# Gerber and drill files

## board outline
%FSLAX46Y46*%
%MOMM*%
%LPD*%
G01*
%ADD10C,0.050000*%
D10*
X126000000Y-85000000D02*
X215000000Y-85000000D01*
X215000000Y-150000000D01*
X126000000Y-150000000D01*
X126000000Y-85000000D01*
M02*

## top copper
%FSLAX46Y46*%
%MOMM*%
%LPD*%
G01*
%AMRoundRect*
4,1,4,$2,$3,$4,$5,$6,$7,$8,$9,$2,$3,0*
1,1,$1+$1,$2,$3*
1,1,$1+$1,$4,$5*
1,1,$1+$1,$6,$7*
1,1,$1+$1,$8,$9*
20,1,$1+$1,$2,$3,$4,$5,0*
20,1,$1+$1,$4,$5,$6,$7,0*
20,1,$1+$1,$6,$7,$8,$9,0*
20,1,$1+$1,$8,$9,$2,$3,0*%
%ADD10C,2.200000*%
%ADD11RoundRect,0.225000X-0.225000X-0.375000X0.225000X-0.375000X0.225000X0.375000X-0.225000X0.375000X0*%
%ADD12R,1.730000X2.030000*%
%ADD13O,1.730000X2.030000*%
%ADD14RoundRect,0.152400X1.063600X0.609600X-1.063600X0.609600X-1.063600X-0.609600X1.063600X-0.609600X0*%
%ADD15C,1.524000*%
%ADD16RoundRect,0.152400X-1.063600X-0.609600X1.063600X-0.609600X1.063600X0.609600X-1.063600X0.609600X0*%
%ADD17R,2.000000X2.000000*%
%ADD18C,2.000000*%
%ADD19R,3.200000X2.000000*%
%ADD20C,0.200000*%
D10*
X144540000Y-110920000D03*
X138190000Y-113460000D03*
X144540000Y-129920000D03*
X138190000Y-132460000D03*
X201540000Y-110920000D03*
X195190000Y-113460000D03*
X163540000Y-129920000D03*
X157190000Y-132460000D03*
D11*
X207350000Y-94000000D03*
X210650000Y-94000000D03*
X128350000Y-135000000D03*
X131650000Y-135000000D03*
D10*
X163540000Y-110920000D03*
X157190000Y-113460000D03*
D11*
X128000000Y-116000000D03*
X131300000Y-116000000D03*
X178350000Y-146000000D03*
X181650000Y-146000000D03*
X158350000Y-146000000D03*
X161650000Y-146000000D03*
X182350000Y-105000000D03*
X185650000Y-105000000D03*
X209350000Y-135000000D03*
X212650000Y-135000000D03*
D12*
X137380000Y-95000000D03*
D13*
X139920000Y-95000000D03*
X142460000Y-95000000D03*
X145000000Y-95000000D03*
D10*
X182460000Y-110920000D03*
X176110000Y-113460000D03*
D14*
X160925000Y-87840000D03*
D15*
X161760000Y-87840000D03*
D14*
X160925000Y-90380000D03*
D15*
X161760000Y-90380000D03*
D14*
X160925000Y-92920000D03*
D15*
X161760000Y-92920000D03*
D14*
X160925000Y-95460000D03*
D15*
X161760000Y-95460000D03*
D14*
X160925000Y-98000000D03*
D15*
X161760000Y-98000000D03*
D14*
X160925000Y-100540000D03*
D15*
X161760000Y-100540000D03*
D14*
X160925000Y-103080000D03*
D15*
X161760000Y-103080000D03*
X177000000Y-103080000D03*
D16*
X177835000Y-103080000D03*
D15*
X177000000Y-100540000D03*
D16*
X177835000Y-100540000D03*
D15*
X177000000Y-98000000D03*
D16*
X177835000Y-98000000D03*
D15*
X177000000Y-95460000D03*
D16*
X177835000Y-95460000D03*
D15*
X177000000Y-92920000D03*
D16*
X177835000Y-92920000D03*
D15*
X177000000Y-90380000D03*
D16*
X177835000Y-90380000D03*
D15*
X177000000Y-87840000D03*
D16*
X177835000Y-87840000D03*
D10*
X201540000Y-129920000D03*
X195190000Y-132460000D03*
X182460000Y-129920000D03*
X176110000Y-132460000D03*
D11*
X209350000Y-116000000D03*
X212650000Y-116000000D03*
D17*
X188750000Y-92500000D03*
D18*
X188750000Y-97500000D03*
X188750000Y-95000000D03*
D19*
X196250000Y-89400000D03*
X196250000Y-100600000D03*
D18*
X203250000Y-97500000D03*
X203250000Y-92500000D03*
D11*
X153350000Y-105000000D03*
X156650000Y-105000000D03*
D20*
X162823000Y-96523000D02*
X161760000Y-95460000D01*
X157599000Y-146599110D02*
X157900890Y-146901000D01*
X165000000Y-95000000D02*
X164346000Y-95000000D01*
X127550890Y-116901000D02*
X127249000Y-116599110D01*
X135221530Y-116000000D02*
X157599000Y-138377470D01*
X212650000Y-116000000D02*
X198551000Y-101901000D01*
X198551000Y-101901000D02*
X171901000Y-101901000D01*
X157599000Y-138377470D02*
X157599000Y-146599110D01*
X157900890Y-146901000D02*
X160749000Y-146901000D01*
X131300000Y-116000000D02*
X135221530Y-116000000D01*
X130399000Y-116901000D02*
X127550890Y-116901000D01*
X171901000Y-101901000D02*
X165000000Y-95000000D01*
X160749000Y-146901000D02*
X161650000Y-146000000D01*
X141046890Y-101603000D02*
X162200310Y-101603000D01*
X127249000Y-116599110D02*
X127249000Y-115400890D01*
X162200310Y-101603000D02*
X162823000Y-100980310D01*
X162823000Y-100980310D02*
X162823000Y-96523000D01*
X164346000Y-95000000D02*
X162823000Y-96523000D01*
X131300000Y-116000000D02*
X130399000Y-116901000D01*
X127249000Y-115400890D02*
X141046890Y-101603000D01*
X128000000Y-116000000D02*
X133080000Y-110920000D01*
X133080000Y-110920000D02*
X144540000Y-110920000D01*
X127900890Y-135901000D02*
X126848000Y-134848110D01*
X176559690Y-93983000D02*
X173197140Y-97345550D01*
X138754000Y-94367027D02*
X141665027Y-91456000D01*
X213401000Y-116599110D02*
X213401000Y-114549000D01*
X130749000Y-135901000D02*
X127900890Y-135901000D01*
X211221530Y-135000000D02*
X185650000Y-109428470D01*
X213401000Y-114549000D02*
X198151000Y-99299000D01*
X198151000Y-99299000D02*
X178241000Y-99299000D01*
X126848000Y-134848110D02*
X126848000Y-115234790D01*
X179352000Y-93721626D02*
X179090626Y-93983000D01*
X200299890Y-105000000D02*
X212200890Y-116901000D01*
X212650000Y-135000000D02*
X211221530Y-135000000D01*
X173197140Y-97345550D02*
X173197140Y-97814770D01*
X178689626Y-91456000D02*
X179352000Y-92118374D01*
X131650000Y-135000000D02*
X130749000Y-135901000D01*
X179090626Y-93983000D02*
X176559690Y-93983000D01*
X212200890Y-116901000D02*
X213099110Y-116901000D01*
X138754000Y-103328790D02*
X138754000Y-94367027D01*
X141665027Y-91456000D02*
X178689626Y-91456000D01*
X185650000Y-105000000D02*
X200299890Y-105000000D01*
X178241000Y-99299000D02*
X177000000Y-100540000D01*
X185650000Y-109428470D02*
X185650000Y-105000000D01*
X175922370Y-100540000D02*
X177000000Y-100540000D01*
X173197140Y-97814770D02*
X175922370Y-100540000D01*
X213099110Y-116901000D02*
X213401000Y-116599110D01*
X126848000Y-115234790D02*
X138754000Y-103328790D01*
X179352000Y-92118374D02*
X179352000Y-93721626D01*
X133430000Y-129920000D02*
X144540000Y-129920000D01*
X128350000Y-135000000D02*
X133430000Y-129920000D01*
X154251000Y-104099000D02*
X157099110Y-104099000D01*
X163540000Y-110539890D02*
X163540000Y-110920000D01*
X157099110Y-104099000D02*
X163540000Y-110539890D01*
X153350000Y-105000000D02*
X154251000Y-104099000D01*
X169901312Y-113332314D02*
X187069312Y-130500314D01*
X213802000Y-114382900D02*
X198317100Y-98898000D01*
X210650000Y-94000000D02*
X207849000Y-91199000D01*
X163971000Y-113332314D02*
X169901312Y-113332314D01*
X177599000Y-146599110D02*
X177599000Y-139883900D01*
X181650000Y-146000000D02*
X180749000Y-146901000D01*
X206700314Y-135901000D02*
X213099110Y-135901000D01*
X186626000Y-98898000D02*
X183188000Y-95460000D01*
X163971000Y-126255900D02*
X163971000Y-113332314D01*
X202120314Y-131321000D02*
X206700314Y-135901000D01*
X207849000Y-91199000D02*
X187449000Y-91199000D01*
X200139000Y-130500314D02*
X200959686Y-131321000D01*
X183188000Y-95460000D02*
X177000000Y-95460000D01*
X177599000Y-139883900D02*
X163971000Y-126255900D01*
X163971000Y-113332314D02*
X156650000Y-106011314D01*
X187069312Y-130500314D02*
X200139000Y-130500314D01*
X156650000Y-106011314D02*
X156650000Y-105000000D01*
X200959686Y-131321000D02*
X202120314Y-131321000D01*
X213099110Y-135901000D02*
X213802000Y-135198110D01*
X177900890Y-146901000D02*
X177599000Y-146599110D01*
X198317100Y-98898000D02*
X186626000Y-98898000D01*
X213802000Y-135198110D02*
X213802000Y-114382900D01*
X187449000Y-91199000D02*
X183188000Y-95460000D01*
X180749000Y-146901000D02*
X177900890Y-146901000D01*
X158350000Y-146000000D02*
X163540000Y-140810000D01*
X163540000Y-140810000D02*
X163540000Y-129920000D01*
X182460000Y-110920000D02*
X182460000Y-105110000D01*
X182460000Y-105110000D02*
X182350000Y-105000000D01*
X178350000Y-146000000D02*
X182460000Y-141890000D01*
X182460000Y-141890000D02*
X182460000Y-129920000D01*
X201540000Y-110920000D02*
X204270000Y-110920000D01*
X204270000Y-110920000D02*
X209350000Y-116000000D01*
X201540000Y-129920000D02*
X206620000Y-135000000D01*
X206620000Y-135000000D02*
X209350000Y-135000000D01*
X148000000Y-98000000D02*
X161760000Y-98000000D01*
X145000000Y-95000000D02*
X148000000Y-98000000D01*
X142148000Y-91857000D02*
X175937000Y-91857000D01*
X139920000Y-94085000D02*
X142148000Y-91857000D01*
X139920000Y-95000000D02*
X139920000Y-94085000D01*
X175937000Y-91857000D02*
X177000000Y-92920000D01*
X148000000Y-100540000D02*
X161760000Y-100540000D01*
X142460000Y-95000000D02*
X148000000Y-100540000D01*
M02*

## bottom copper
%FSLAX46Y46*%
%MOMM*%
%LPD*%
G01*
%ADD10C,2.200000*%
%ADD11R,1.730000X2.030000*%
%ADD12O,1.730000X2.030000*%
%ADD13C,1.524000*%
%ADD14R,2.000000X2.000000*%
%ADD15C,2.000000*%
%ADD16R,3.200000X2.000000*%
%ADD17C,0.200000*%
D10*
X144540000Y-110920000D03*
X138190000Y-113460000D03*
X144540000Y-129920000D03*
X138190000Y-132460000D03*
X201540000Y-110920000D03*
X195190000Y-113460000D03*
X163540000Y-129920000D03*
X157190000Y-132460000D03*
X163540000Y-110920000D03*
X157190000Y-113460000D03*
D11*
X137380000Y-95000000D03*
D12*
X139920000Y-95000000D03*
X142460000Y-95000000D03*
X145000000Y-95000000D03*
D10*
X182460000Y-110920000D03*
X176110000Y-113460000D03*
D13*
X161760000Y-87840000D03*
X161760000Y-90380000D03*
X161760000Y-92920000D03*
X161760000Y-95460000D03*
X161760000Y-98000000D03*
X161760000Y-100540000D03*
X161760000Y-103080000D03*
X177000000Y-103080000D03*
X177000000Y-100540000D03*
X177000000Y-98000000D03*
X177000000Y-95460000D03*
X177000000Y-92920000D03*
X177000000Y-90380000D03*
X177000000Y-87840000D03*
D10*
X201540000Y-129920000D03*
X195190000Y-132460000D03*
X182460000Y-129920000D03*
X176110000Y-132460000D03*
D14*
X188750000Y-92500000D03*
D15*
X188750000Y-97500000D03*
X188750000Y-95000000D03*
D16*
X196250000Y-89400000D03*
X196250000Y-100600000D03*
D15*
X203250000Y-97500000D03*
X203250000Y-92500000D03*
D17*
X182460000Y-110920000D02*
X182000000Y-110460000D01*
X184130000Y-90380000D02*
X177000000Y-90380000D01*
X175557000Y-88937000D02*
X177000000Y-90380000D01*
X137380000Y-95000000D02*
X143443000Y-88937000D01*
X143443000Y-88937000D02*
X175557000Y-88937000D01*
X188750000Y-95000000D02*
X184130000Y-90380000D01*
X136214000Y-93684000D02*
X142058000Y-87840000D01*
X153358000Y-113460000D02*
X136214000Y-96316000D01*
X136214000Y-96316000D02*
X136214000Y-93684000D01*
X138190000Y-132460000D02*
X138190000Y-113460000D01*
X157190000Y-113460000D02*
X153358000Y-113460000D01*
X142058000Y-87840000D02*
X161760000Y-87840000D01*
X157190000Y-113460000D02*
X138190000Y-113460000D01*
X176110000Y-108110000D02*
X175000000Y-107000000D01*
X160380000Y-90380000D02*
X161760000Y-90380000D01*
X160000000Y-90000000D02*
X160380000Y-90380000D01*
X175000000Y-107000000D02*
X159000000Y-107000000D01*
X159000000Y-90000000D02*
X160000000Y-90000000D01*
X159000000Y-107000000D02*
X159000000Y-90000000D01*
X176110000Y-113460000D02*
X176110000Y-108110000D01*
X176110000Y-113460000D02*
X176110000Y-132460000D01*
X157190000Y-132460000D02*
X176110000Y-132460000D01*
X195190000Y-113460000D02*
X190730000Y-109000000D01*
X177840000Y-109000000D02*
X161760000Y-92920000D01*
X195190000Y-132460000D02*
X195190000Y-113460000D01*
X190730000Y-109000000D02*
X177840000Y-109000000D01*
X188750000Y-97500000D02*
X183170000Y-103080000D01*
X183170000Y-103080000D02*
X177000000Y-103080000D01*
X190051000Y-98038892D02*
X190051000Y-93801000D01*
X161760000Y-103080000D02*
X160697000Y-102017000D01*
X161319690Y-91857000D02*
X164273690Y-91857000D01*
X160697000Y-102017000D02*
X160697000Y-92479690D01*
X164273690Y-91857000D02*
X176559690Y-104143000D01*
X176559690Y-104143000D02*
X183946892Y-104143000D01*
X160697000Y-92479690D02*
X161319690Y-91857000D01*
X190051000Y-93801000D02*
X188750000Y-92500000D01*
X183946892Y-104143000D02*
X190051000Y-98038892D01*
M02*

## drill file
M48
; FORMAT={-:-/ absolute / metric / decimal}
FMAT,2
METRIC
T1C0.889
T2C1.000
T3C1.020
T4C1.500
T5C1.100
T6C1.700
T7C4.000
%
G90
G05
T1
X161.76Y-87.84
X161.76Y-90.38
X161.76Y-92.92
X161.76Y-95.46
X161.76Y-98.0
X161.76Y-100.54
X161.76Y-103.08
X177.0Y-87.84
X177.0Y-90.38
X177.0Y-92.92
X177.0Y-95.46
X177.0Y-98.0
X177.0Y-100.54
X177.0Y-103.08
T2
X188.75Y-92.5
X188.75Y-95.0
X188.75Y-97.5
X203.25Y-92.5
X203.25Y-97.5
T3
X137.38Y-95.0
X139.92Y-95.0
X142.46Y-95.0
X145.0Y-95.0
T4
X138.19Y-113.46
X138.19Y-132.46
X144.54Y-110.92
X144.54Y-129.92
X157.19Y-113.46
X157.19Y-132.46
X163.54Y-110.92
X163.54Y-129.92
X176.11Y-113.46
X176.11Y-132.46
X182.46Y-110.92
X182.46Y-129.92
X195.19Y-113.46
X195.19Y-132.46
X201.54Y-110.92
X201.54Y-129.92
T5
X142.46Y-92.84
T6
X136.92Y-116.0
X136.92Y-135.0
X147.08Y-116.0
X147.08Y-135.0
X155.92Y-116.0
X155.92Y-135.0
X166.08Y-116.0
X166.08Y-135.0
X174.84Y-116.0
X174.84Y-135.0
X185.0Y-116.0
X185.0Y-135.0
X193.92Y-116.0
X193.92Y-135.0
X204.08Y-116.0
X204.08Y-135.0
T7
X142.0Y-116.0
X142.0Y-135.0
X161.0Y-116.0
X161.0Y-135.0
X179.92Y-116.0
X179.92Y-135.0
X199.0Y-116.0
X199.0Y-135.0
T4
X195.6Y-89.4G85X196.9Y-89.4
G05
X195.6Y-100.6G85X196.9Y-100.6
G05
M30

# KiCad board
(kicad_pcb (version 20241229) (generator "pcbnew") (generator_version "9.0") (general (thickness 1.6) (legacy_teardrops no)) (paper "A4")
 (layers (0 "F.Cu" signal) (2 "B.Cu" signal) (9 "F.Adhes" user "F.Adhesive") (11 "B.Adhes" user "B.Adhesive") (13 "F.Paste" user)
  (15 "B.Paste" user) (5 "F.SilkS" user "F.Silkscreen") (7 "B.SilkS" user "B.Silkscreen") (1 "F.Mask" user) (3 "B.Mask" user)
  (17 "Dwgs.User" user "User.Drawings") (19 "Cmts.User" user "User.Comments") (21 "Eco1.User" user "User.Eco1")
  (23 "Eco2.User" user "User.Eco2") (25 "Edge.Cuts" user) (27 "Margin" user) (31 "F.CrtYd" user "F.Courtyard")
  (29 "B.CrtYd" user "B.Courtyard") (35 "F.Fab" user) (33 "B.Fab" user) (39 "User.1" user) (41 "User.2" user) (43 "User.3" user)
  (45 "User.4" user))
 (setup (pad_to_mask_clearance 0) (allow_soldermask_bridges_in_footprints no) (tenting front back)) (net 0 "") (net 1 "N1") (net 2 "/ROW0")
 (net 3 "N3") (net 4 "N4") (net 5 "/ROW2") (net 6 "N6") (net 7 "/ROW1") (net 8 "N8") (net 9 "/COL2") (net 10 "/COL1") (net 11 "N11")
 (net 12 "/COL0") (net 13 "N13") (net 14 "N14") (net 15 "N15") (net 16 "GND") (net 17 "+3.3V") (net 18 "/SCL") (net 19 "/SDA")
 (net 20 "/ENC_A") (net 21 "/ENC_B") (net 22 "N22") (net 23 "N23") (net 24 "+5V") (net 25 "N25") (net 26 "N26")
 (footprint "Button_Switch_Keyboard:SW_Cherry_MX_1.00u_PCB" (layer "F.Cu") (at 144.54 110.92)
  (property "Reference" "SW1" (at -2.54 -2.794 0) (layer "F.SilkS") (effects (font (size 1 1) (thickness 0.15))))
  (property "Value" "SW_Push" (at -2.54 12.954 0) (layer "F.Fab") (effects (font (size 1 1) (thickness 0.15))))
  (pad "" np_thru_hole circle (at -7.62 5.08) (size 1.7 1.7) (drill 1.7) (layers "*.Cu" "*.Mask"))
  (pad "" np_thru_hole circle (at -2.54 5.08) (size 4 4) (drill 4) (layers "*.Cu" "*.Mask"))
  (pad "" np_thru_hole circle (at 2.54 5.08) (size 1.7 1.7) (drill 1.7) (layers "*.Cu" "*.Mask"))
  (pad "1" thru_hole circle (at 0 0) (size 2.2 2.2) (drill 1.5) (layers "*.Cu" "*.Mask") (remove_unused_layers no) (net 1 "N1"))
  (pad "2" thru_hole circle (at -6.35 2.54) (size 2.2 2.2) (drill 1.5) (layers "*.Cu" "*.Mask") (remove_unused_layers no) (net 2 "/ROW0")))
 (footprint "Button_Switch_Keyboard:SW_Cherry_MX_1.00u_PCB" (layer "F.Cu") (at 144.54 129.92)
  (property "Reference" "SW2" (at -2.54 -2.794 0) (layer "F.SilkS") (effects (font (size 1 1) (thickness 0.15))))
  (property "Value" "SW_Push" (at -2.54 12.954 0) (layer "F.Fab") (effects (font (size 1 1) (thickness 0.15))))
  (pad "" np_thru_hole circle (at -7.62 5.08) (size 1.7 1.7) (drill 1.7) (layers "*.Cu" "*.Mask"))
  (pad "" np_thru_hole circle (at -2.54 5.08) (size 4 4) (drill 4) (layers "*.Cu" "*.Mask"))
  (pad "" np_thru_hole circle (at 2.54 5.08) (size 1.7 1.7) (drill 1.7) (layers "*.Cu" "*.Mask"))
  (pad "1" thru_hole circle (at 0 0) (size 2.2 2.2) (drill 1.5) (layers "*.Cu" "*.Mask") (remove_unused_layers no) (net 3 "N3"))
  (pad "2" thru_hole circle (at -6.35 2.54) (size 2.2 2.2) (drill 1.5) (layers "*.Cu" "*.Mask") (remove_unused_layers no) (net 2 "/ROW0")))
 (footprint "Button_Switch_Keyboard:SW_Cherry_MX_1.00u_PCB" (layer "F.Cu") (at 201.54 110.92)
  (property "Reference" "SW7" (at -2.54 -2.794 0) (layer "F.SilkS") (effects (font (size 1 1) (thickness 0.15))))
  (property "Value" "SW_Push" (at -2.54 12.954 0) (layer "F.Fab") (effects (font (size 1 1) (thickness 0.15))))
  (pad "" np_thru_hole circle (at -7.62 5.08) (size 1.7 1.7) (drill 1.7) (layers "*.Cu" "*.Mask"))
  (pad "" np_thru_hole circle (at -2.54 5.08) (size 4 4) (drill 4) (layers "*.Cu" "*.Mask"))
  (pad "" np_thru_hole circle (at 2.54 5.08) (size 1.7 1.7) (drill 1.7) (layers "*.Cu" "*.Mask"))
  (pad "1" thru_hole circle (at 0 0) (size 2.2 2.2) (drill 1.5) (layers "*.Cu" "*.Mask") (remove_unused_layers no) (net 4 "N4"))
  (pad "2" thru_hole circle (at -6.35 2.54) (size 2.2 2.2) (drill 1.5) (layers "*.Cu" "*.Mask") (remove_unused_layers no) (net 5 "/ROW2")))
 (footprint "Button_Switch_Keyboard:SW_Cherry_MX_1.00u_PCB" (layer "F.Cu") (at 163.54 129.92)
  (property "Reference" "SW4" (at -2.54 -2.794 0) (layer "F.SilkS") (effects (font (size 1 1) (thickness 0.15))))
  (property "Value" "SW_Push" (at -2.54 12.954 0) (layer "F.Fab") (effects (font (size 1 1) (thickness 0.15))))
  (pad "" np_thru_hole circle (at -7.62 5.08) (size 1.7 1.7) (drill 1.7) (layers "*.Cu" "*.Mask"))
  (pad "" np_thru_hole circle (at -2.54 5.08) (size 4 4) (drill 4) (layers "*.Cu" "*.Mask"))
  (pad "" np_thru_hole circle (at 2.54 5.08) (size 1.7 1.7) (drill 1.7) (layers "*.Cu" "*.Mask"))
  (pad "1" thru_hole circle (at 0 0) (size 2.2 2.2) (drill 1.5) (layers "*.Cu" "*.Mask") (remove_unused_layers no) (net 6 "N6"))
  (pad "2" thru_hole circle (at -6.35 2.54) (size 2.2 2.2) (drill 1.5) (layers "*.Cu" "*.Mask") (remove_unused_layers no) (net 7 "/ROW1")))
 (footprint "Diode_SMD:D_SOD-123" (layer "F.Cu") (at 209 94)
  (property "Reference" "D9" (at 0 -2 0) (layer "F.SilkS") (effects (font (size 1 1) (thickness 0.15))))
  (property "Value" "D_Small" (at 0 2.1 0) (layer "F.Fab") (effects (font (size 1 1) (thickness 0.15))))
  (pad "1" smd roundrect (at -1.65 0) (size 0.9 1.2) (layers "F.Cu" "F.Mask" "F.Paste") (roundrect_rratio 0.25) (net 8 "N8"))
  (pad "2" smd roundrect (at 1.65 0) (size 0.9 1.2) (layers "F.Cu" "F.Mask" "F.Paste") (roundrect_rratio 0.25) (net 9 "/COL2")))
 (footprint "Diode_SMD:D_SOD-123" (layer "F.Cu") (at 130 135)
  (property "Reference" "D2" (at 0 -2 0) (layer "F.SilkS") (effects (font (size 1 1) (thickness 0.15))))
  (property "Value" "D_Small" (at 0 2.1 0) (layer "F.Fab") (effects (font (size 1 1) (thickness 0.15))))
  (pad "1" smd roundrect (at -1.65 0) (size 0.9 1.2) (layers "F.Cu" "F.Mask" "F.Paste") (roundrect_rratio 0.25) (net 3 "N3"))
  (pad "2" smd roundrect (at 1.65 0) (size 0.9 1.2) (layers "F.Cu" "F.Mask" "F.Paste") (roundrect_rratio 0.25) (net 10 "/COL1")))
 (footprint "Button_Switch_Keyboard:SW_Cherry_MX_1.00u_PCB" (layer "F.Cu") (at 163.54 110.92)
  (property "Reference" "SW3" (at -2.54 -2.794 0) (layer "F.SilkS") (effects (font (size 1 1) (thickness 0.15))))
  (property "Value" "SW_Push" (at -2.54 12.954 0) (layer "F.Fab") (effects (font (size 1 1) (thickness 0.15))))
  (pad "" np_thru_hole circle (at -7.62 5.08) (size 1.7 1.7) (drill 1.7) (layers "*.Cu" "*.Mask"))
  (pad "" np_thru_hole circle (at -2.54 5.08) (size 4 4) (drill 4) (layers "*.Cu" "*.Mask"))
  (pad "" np_thru_hole circle (at 2.54 5.08) (size 1.7 1.7) (drill 1.7) (layers "*.Cu" "*.Mask"))
  (pad "1" thru_hole circle (at 0 0) (size 2.2 2.2) (drill 1.5) (layers "*.Cu" "*.Mask") (remove_unused_layers no) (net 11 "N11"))
  (pad "2" thru_hole circle (at -6.35 2.54) (size 2.2 2.2) (drill 1.5) (layers "*.Cu" "*.Mask") (remove_unused_layers no) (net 2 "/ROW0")))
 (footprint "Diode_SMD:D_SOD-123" (layer "F.Cu") (at 129.65 116)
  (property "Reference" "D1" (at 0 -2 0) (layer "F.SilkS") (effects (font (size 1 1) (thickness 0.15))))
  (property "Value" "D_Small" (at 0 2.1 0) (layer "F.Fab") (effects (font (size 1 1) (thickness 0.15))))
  (pad "1" smd roundrect (at -1.65 0) (size 0.9 1.2) (layers "F.Cu" "F.Mask" "F.Paste") (roundrect_rratio 0.25) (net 1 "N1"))
  (pad "2" smd roundrect (at 1.65 0) (size 0.9 1.2) (layers "F.Cu" "F.Mask" "F.Paste") (roundrect_rratio 0.25) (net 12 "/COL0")))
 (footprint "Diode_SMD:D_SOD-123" (layer "F.Cu") (at 180 146)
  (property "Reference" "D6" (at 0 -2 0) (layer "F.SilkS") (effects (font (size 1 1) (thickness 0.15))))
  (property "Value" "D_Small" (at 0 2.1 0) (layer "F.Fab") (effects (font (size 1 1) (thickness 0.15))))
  (pad "1" smd roundrect (at -1.65 0) (size 0.9 1.2) (layers "F.Cu" "F.Mask" "F.Paste") (roundrect_rratio 0.25) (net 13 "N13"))
  (pad "2" smd roundrect (at 1.65 0) (size 0.9 1.2) (layers "F.Cu" "F.Mask" "F.Paste") (roundrect_rratio 0.25) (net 9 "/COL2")))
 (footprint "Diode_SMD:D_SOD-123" (layer "F.Cu") (at 160 146)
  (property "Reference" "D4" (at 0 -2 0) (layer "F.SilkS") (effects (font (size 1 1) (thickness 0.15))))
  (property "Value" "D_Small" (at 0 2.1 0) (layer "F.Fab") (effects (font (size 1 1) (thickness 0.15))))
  (pad "1" smd roundrect (at -1.65 0) (size 0.9 1.2) (layers "F.Cu" "F.Mask" "F.Paste") (roundrect_rratio 0.25) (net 6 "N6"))
  (pad "2" smd roundrect (at 1.65 0) (size 0.9 1.2) (layers "F.Cu" "F.Mask" "F.Paste") (roundrect_rratio 0.25) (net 12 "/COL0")))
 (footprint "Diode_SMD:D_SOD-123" (layer "F.Cu") (at 184 105)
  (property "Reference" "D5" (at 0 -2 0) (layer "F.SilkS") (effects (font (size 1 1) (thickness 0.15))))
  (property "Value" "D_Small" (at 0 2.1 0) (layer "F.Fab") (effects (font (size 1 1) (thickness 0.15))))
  (pad "1" smd roundrect (at -1.65 0) (size 0.9 1.2) (layers "F.Cu" "F.Mask" "F.Paste") (roundrect_rratio 0.25) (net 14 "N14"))
  (pad "2" smd roundrect (at 1.65 0) (size 0.9 1.2) (layers "F.Cu" "F.Mask" "F.Paste") (roundrect_rratio 0.25) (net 10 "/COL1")))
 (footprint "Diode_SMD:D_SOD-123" (layer "F.Cu") (at 211 135)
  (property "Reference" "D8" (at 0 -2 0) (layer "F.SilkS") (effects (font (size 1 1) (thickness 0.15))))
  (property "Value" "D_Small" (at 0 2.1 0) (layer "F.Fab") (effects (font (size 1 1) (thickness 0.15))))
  (pad "1" smd roundrect (at -1.65 0) (size 0.9 1.2) (layers "F.Cu" "F.Mask" "F.Paste") (roundrect_rratio 0.25) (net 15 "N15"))
  (pad "2" smd roundrect (at 1.65 0) (size 0.9 1.2) (layers "F.Cu" "F.Mask" "F.Paste") (roundrect_rratio 0.25) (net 10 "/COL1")))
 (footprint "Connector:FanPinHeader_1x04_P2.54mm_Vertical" (layer "F.Cu") (at 137.38 95)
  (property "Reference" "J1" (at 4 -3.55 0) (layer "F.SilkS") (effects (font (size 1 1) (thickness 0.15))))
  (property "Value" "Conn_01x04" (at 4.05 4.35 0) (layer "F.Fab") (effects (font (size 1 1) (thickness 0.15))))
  (pad "" np_thru_hole circle (at 5.08 -2.16 90) (size 1.1 1.1) (drill 1.1) (layers "*.Cu" "*.Mask"))
  (pad "1" thru_hole rect (at 0 0 90) (size 2.03 1.73) (drill 1.02) (layers "*.Cu" "*.Mask") (remove_unused_layers no) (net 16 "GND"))
  (pad "2" thru_hole oval (at 2.54 0 90) (size 2.03 1.73) (drill 1.02) (layers "*.Cu" "*.Mask") (remove_unused_layers no) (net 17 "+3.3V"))
  (pad "3" thru_hole oval (at 5.08 0 90) (size 2.03 1.73) (drill 1.02) (layers "*.Cu" "*.Mask") (remove_unused_layers no) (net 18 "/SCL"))
  (pad "4" thru_hole oval (at 7.62 0 90) (size 2.03 1.73) (drill 1.02) (layers "*.Cu" "*.Mask") (remove_unused_layers no) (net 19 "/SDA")))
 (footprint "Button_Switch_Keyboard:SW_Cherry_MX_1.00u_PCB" (layer "F.Cu") (at 182.46 110.92)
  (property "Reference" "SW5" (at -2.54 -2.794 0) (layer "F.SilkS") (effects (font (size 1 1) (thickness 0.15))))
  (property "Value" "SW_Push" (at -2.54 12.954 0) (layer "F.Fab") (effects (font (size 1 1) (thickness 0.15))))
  (pad "" np_thru_hole circle (at -7.62 5.08) (size 1.7 1.7) (drill 1.7) (layers "*.Cu" "*.Mask"))
  (pad "" np_thru_hole circle (at -2.54 5.08) (size 4 4) (drill 4) (layers "*.Cu" "*.Mask"))
  (pad "" np_thru_hole circle (at 2.54 5.08) (size 1.7 1.7) (drill 1.7) (layers "*.Cu" "*.Mask"))
  (pad "1" thru_hole circle (at 0 0) (size 2.2 2.2) (drill 1.5) (layers "*.Cu" "*.Mask") (remove_unused_layers no) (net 14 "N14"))
  (pad "2" thru_hole circle (at -6.35 2.54) (size 2.2 2.2) (drill 1.5) (layers "*.Cu" "*.Mask") (remove_unused_layers no) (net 7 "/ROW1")))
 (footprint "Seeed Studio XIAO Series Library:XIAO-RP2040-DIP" (layer "F.Cu") (at 169.38 95.46)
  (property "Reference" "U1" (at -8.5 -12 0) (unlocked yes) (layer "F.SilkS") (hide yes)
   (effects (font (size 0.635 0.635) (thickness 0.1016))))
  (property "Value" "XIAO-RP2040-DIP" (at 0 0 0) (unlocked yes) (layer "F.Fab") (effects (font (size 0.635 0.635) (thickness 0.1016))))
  (pad "1" smd roundrect (at -8.455 -7.62 180) (size 2.432 1.524) (layers "F.Cu" "F.Mask") (roundrect_rratio 0.1) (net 2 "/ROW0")
   (thermal_bridge_angle 45))
  (pad "1" thru_hole circle (at -7.62 -7.62 180) (size 1.524 1.524) (drill 0.889) (layers "*.Cu" "*.Mask") (remove_unused_layers no)
   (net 2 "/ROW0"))
  (pad "2" smd roundrect (at -8.455 -5.08 180) (size 2.432 1.524) (layers "F.Cu" "F.Mask") (roundrect_rratio 0.1) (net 7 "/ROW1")
   (thermal_bridge_angle 45))
  (pad "2" thru_hole circle (at -7.62 -5.08 180) (size 1.524 1.524) (drill 0.889) (layers "*.Cu" "*.Mask") (remove_unused_layers no)
   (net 7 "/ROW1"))
  (pad "3" smd roundrect (at -8.455 -2.54 180) (size 2.432 1.524) (layers "F.Cu" "F.Mask") (roundrect_rratio 0.1) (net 5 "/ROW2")
   (thermal_bridge_angle 45))
  (pad "3" thru_hole circle (at -7.62 -2.54 180) (size 1.524 1.524) (drill 0.889) (layers "*.Cu" "*.Mask") (remove_unused_layers no)
   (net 5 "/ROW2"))
  (pad "4" smd roundrect (at -8.455 0 180) (size 2.432 1.524) (layers "F.Cu" "F.Mask") (roundrect_rratio 0.1) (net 12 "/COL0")
   (thermal_bridge_angle 45))
  (pad "4" thru_hole circle (at -7.62 0 180) (size 1.524 1.524) (drill 0.889) (layers "*.Cu" "*.Mask") (remove_unused_layers no)
   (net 12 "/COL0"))
  (pad "5" smd roundrect (at -8.455 2.54 180) (size 2.432 1.524) (layers "F.Cu" "F.Mask") (roundrect_rratio 0.1) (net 19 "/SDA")
   (thermal_bridge_angle 45))
  (pad "5" thru_hole circle (at -7.62 2.54 180) (size 1.524 1.524) (drill 0.889) (layers "*.Cu" "*.Mask") (remove_unused_layers no)
   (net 19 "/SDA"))
  (pad "6" smd roundrect (at -8.455 5.08 180) (size 2.432 1.524) (layers "F.Cu" "F.Mask") (roundrect_rratio 0.1) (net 18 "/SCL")
   (thermal_bridge_angle 45))
  (pad "6" thru_hole circle (at -7.62 5.08 180) (size 1.524 1.524) (drill 0.889) (layers "*.Cu" "*.Mask") (remove_unused_layers no)
   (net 18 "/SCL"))
  (pad "7" smd roundrect (at -8.455 7.62 180) (size 2.432 1.524) (layers "F.Cu" "F.Mask") (roundrect_rratio 0.1) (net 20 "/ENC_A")
   (thermal_bridge_angle 45))
  (pad "7" thru_hole circle (at -7.62 7.62 180) (size 1.524 1.524) (drill 0.889) (layers "*.Cu" "*.Mask") (remove_unused_layers no)
   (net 20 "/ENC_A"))
  (pad "8" thru_hole circle (at 7.62 7.62) (size 1.524 1.524) (drill 0.889) (layers "*.Cu" "*.Mask") (remove_unused_layers no)
   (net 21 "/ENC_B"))
  (pad "8" smd roundrect (at 8.455 7.62) (size 2.432 1.524) (layers "F.Cu" "F.Mask") (roundrect_rratio 0.1) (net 21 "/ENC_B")
   (thermal_bridge_angle 45))
  (pad "9" thru_hole circle (at 7.62 5.08) (size 1.524 1.524) (drill 0.889) (layers "*.Cu" "*.Mask") (remove_unused_layers no)
   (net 10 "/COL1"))
  (pad "9" smd roundrect (at 8.455 5.08) (size 2.432 1.524) (layers "F.Cu" "F.Mask") (roundrect_rratio 0.1) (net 10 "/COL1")
   (thermal_bridge_angle 45))
  (pad "10" thru_hole circle (at 7.62 2.54) (size 1.524 1.524) (drill 0.889) (layers "*.Cu" "*.Mask") (remove_unused_layers no)
   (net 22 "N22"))
  (pad "10" smd roundrect (at 8.455 2.54) (size 2.432 1.524) (layers "F.Cu" "F.Mask") (roundrect_rratio 0.1) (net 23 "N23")
   (thermal_bridge_angle 45))
  (pad "11" thru_hole circle (at 7.62 0) (size 1.524 1.524) (drill 0.889) (layers "*.Cu" "*.Mask") (remove_unused_layers no) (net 9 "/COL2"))
  (pad "11" smd roundrect (at 8.455 0) (size 2.432 1.524) (layers "F.Cu" "F.Mask") (roundrect_rratio 0.1) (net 9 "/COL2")
   (thermal_bridge_angle 45))
  (pad "12" thru_hole circle (at 7.62 -2.54) (size 1.524 1.524) (drill 0.889) (layers "*.Cu" "*.Mask") (remove_unused_layers no)
   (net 17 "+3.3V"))
  (pad "12" smd roundrect (at 8.455 -2.54) (size 2.432 1.524) (layers "F.Cu" "F.Mask") (roundrect_rratio 0.1) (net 17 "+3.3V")
   (thermal_bridge_angle 45))
  (pad "13" thru_hole circle (at 7.62 -5.08) (size 1.524 1.524) (drill 0.889) (layers "*.Cu" "*.Mask") (remove_unused_layers no)
   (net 16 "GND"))
  (pad "13" smd roundrect (at 8.455 -5.08) (size 2.432 1.524) (layers "F.Cu" "F.Mask") (roundrect_rratio 0.1) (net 16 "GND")
   (thermal_bridge_angle 45))
  (pad "14" thru_hole circle (at 7.62 -7.62) (size 1.524 1.524) (drill 0.889) (layers "*.Cu" "*.Mask") (remove_unused_layers no)
   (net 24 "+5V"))
  (pad "14" smd roundrect (at 8.455 -7.62) (size 2.432 1.524) (layers "F.Cu" "F.Mask") (roundrect_rratio 0.1) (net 24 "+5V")
   (thermal_bridge_angle 45)))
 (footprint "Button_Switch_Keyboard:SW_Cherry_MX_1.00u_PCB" (layer "F.Cu") (at 201.54 129.92)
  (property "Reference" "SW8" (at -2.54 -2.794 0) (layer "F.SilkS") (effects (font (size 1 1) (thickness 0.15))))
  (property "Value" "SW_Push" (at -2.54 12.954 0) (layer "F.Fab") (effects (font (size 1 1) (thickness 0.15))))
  (pad "" np_thru_hole circle (at -7.62 5.08) (size 1.7 1.7) (drill 1.7) (layers "*.Cu" "*.Mask"))
  (pad "" np_thru_hole circle (at -2.54 5.08) (size 4 4) (drill 4) (layers "*.Cu" "*.Mask"))
  (pad "" np_thru_hole circle (at 2.54 5.08) (size 1.7 1.7) (drill 1.7) (layers "*.Cu" "*.Mask"))
  (pad "1" thru_hole circle (at 0 0) (size 2.2 2.2) (drill 1.5) (layers "*.Cu" "*.Mask") (remove_unused_layers no) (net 15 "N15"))
  (pad "2" thru_hole circle (at -6.35 2.54) (size 2.2 2.2) (drill 1.5) (layers "*.Cu" "*.Mask") (remove_unused_layers no) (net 5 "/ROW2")))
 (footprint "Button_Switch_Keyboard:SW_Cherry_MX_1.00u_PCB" (layer "F.Cu") (at 182.46 129.92)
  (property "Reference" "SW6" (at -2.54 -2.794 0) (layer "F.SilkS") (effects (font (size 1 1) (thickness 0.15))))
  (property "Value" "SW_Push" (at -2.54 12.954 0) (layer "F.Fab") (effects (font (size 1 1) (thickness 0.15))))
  (pad "" np_thru_hole circle (at -7.62 5.08) (size 1.7 1.7) (drill 1.7) (layers "*.Cu" "*.Mask"))
  (pad "" np_thru_hole circle (at -2.54 5.08) (size 4 4) (drill 4) (layers "*.Cu" "*.Mask"))
  (pad "" np_thru_hole circle (at 2.54 5.08) (size 1.7 1.7) (drill 1.7) (layers "*.Cu" "*.Mask"))
  (pad "1" thru_hole circle (at 0 0) (size 2.2 2.2) (drill 1.5) (layers "*.Cu" "*.Mask") (remove_unused_layers no) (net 13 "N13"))
  (pad "2" thru_hole circle (at -6.35 2.54) (size 2.2 2.2) (drill 1.5) (layers "*.Cu" "*.Mask") (remove_unused_layers no) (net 7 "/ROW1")))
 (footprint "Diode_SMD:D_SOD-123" (layer "F.Cu") (at 211 116)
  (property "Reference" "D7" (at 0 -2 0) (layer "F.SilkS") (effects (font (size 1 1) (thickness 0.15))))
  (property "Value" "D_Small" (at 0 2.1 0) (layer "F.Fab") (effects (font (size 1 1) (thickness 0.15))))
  (pad "1" smd roundrect (at -1.65 0) (size 0.9 1.2) (layers "F.Cu" "F.Mask" "F.Paste") (roundrect_rratio 0.25) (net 4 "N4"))
  (pad "2" smd roundrect (at 1.65 0) (size 0.9 1.2) (layers "F.Cu" "F.Mask" "F.Paste") (roundrect_rratio 0.25) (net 12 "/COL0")))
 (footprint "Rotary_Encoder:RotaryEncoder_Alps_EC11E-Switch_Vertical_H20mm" (layer "F.Cu") (at 188.75 92.5)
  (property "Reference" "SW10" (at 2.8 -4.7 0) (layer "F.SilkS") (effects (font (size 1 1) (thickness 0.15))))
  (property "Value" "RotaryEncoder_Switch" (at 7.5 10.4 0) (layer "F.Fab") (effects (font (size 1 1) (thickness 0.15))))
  (pad "A" thru_hole rect (at 0 0) (size 2 2) (drill 1) (layers "*.Cu" "*.Mask") (remove_unused_layers no) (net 20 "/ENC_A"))
  (pad "B" thru_hole circle (at 0 5) (size 2 2) (drill 1) (layers "*.Cu" "*.Mask") (remove_unused_layers no) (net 21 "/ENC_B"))
  (pad "C" thru_hole circle (at 0 2.5) (size 2 2) (drill 1) (layers "*.Cu" "*.Mask") (remove_unused_layers no) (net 16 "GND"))
  (pad "MP" thru_hole rect (at 7.5 -3.1) (size 3.2 2) (drill oval 2.8 1.5) (layers "*.Cu" "*.Mask") (remove_unused_layers no))
  (pad "MP" thru_hole rect (at 7.5 8.1) (size 3.2 2) (drill oval 2.8 1.5) (layers "*.Cu" "*.Mask") (remove_unused_layers no))
  (pad "S1" thru_hole circle (at 14.5 5) (size 2 2) (drill 1) (layers "*.Cu" "*.Mask") (remove_unused_layers no) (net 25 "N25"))
  (pad "S2" thru_hole circle (at 14.5 0) (size 2 2) (drill 1) (layers "*.Cu" "*.Mask") (remove_unused_layers no) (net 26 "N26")))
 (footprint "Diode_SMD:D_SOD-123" (layer "F.Cu") (at 155 105)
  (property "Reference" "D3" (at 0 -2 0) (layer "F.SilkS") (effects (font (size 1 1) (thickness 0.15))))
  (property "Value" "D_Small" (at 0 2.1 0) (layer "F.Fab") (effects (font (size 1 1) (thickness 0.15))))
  (pad "1" smd roundrect (at -1.65 0) (size 0.9 1.2) (layers "F.Cu" "F.Mask" "F.Paste") (roundrect_rratio 0.25) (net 11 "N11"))
  (pad "2" smd roundrect (at 1.65 0) (size 0.9 1.2) (layers "F.Cu" "F.Mask" "F.Paste") (roundrect_rratio 0.25) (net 9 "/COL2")))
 (gr_rect (start 126 85) (end 215 150) (stroke (width 0.05) (type default)) (fill no) (layer "Edge.Cuts"))
 (segment (start 162.823 96.523) (end 161.76 95.46) (width 0.2) (layer "F.Cu") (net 12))
 (segment (start 157.599 146.59911) (end 157.90089 146.901) (width 0.2) (layer "F.Cu") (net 12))
 (segment (start 165 95) (end 164.346 95) (width 0.2) (layer "F.Cu") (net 12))
 (segment (start 127.55089 116.901) (end 127.249 116.59911) (width 0.2) (layer "F.Cu") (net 12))
 (segment (start 135.22153 116) (end 157.599 138.37747) (width 0.2) (layer "F.Cu") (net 12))
 (segment (start 212.65 116) (end 198.551 101.901) (width 0.2) (layer "F.Cu") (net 12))
 (segment (start 198.551 101.901) (end 171.901 101.901) (width 0.2) (layer "F.Cu") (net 12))
 (segment (start 157.599 138.37747) (end 157.599 146.59911) (width 0.2) (layer "F.Cu") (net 12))
 (segment (start 157.90089 146.901) (end 160.749 146.901) (width 0.2) (layer "F.Cu") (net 12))
 (segment (start 131.3 116) (end 135.22153 116) (width 0.2) (layer "F.Cu") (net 12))
 (segment (start 130.399 116.901) (end 127.55089 116.901) (width 0.2) (layer "F.Cu") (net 12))
 (segment (start 171.901 101.901) (end 165 95) (width 0.2) (layer "F.Cu") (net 12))
 (segment (start 160.749 146.901) (end 161.65 146) (width 0.2) (layer "F.Cu") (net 12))
 (segment (start 141.04689 101.603) (end 162.20031 101.603) (width 0.2) (layer "F.Cu") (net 12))
 (segment (start 127.249 116.59911) (end 127.249 115.40089) (width 0.2) (layer "F.Cu") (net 12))
 (segment (start 162.20031 101.603) (end 162.823 100.98031) (width 0.2) (layer "F.Cu") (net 12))
 (segment (start 162.823 100.98031) (end 162.823 96.523) (width 0.2) (layer "F.Cu") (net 12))
 (segment (start 164.346 95) (end 162.823 96.523) (width 0.2) (layer "F.Cu") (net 12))
 (segment (start 131.3 116) (end 130.399 116.901) (width 0.2) (layer "F.Cu") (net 12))
 (segment (start 127.249 115.40089) (end 141.04689 101.603) (width 0.2) (layer "F.Cu") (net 12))
 (segment (start 128 116) (end 133.08 110.92) (width 0.2) (layer "F.Cu") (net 1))
 (segment (start 133.08 110.92) (end 144.54 110.92) (width 0.2) (layer "F.Cu") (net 1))
 (segment (start 127.90089 135.901) (end 126.848 134.84811) (width 0.2) (layer "F.Cu") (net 10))
 (segment (start 176.55969 93.983) (end 173.19714 97.34555) (width 0.2) (layer "F.Cu") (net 10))
 (segment (start 138.754 94.367027) (end 141.665027 91.456) (width 0.2) (layer "F.Cu") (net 10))
 (segment (start 213.401 116.59911) (end 213.401 114.549) (width 0.2) (layer "F.Cu") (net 10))
 (segment (start 130.749 135.901) (end 127.90089 135.901) (width 0.2) (layer "F.Cu") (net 10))
 (segment (start 211.22153 135) (end 185.65 109.42847) (width 0.2) (layer "F.Cu") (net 10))
 (segment (start 213.401 114.549) (end 198.151 99.299) (width 0.2) (layer "F.Cu") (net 10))
 (segment (start 198.151 99.299) (end 178.241 99.299) (width 0.2) (layer "F.Cu") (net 10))
 (segment (start 126.848 134.84811) (end 126.848 115.23479) (width 0.2) (layer "F.Cu") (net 10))
 (segment (start 179.352 93.721626) (end 179.090626 93.983) (width 0.2) (layer "F.Cu") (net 10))
 (segment (start 200.29989 105) (end 212.20089 116.901) (width 0.2) (layer "F.Cu") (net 10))
 (segment (start 212.65 135) (end 211.22153 135) (width 0.2) (layer "F.Cu") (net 10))
 (segment (start 173.19714 97.34555) (end 173.19714 97.81477) (width 0.2) (layer "F.Cu") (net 10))
 (segment (start 178.689626 91.456) (end 179.352 92.118374) (width 0.2) (layer "F.Cu") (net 10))
 (segment (start 131.65 135) (end 130.749 135.901) (width 0.2) (layer "F.Cu") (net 10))
 (segment (start 179.090626 93.983) (end 176.55969 93.983) (width 0.2) (layer "F.Cu") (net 10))
 (segment (start 212.20089 116.901) (end 213.09911 116.901) (width 0.2) (layer "F.Cu") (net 10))
 (segment (start 138.754 103.32879) (end 138.754 94.367027) (width 0.2) (layer "F.Cu") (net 10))
 (segment (start 141.665027 91.456) (end 178.689626 91.456) (width 0.2) (layer "F.Cu") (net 10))
 (segment (start 185.65 105) (end 200.29989 105) (width 0.2) (layer "F.Cu") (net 10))
 (segment (start 178.241 99.299) (end 177 100.54) (width 0.2) (layer "F.Cu") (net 10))
 (segment (start 185.65 109.42847) (end 185.65 105) (width 0.2) (layer "F.Cu") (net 10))
 (segment (start 175.92237 100.54) (end 177 100.54) (width 0.2) (layer "F.Cu") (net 10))
 (segment (start 173.19714 97.81477) (end 175.92237 100.54) (width 0.2) (layer "F.Cu") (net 10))
 (segment (start 213.09911 116.901) (end 213.401 116.59911) (width 0.2) (layer "F.Cu") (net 10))
 (segment (start 126.848 115.23479) (end 138.754 103.32879) (width 0.2) (layer "F.Cu") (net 10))
 (segment (start 179.352 92.118374) (end 179.352 93.721626) (width 0.2) (layer "F.Cu") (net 10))
 (segment (start 133.43 129.92) (end 144.54 129.92) (width 0.2) (layer "F.Cu") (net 3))
 (segment (start 128.35 135) (end 133.43 129.92) (width 0.2) (layer "F.Cu") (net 3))
 (segment (start 154.251 104.099) (end 157.09911 104.099) (width 0.2) (layer "F.Cu") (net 11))
 (segment (start 163.54 110.53989) (end 163.54 110.92) (width 0.2) (layer "F.Cu") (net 11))
 (segment (start 157.09911 104.099) (end 163.54 110.53989) (width 0.2) (layer "F.Cu") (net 11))
 (segment (start 153.35 105) (end 154.251 104.099) (width 0.2) (layer "F.Cu") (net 11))
 (segment (start 169.901312 113.332314) (end 187.069312 130.500314) (width 0.2) (layer "F.Cu") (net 9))
 (segment (start 213.802 114.3829) (end 198.3171 98.898) (width 0.2) (layer "F.Cu") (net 9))
 (segment (start 210.65 94) (end 207.849 91.199) (width 0.2) (layer "F.Cu") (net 9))
 (segment (start 163.971 113.332314) (end 169.901312 113.332314) (width 0.2) (layer "F.Cu") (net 9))
 (segment (start 177.599 146.59911) (end 177.599 139.8839) (width 0.2) (layer "F.Cu") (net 9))
 (segment (start 181.65 146) (end 180.749 146.901) (width 0.2) (layer "F.Cu") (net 9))
 (segment (start 206.700314 135.901) (end 213.09911 135.901) (width 0.2) (layer "F.Cu") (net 9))
 (segment (start 186.626 98.898) (end 183.188 95.46) (width 0.2) (layer "F.Cu") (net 9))
 (segment (start 163.971 126.2559) (end 163.971 113.332314) (width 0.2) (layer "F.Cu") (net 9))
 (segment (start 202.120314 131.321) (end 206.700314 135.901) (width 0.2) (layer "F.Cu") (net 9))
 (segment (start 207.849 91.199) (end 187.449 91.199) (width 0.2) (layer "F.Cu") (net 9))
 (segment (start 200.139 130.500314) (end 200.959686 131.321) (width 0.2) (layer "F.Cu") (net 9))
 (segment (start 183.188 95.46) (end 177 95.46) (width 0.2) (layer "F.Cu") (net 9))
 (segment (start 177.599 139.8839) (end 163.971 126.2559) (width 0.2) (layer "F.Cu") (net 9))
 (segment (start 163.971 113.332314) (end 156.65 106.011314) (width 0.2) (layer "F.Cu") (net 9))
 (segment (start 187.069312 130.500314) (end 200.139 130.500314) (width 0.2) (layer "F.Cu") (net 9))
 (segment (start 156.65 106.011314) (end 156.65 105) (width 0.2) (layer "F.Cu") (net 9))
 (segment (start 200.959686 131.321) (end 202.120314 131.321) (width 0.2) (layer "F.Cu") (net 9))
 (segment (start 213.09911 135.901) (end 213.802 135.19811) (width 0.2) (layer "F.Cu") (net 9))
 (segment (start 177.90089 146.901) (end 177.599 146.59911) (width 0.2) (layer "F.Cu") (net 9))
 (segment (start 198.3171 98.898) (end 186.626 98.898) (width 0.2) (layer "F.Cu") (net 9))
 (segment (start 213.802 135.19811) (end 213.802 114.3829) (width 0.2) (layer "F.Cu") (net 9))
 (segment (start 187.449 91.199) (end 183.188 95.46) (width 0.2) (layer "F.Cu") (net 9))
 (segment (start 180.749 146.901) (end 177.90089 146.901) (width 0.2) (layer "F.Cu") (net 9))
 (segment (start 158.35 146) (end 163.54 140.81) (width 0.2) (layer "F.Cu") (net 6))
 (segment (start 163.54 140.81) (end 163.54 129.92) (width 0.2) (layer "F.Cu") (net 6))
 (segment (start 182.46 110.92) (end 182.46 105.11) (width 0.2) (layer "F.Cu") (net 14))
 (segment (start 182.46 105.11) (end 182.35 105) (width 0.2) (layer "F.Cu") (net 14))
 (segment (start 182.46 110.92) (end 182 110.46) (width 0.2) (layer "B.Cu") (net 14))
 (segment (start 178.35 146) (end 182.46 141.89) (width 0.2) (layer "F.Cu") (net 13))
 (segment (start 182.46 141.89) (end 182.46 129.92) (width 0.2) (layer "F.Cu") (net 13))
 (segment (start 201.54 110.92) (end 204.27 110.92) (width 0.2) (layer "F.Cu") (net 4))
 (segment (start 204.27 110.92) (end 209.35 116) (width 0.2) (layer "F.Cu") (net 4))
 (segment (start 201.54 129.92) (end 206.62 135) (width 0.2) (layer "F.Cu") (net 15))
 (segment (start 206.62 135) (end 209.35 135) (width 0.2) (layer "F.Cu") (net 15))
 (segment (start 148 98) (end 161.76 98) (width 0.2) (layer "F.Cu") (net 19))
 (segment (start 145 95) (end 148 98) (width 0.2) (layer "F.Cu") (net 19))
 (segment (start 142.148 91.857) (end 175.937 91.857) (width 0.2) (layer "F.Cu") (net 17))
 (segment (start 139.92 94.085) (end 142.148 91.857) (width 0.2) (layer "F.Cu") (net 17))
 (segment (start 139.92 95) (end 139.92 94.085) (width 0.2) (layer "F.Cu") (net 17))
 (segment (start 175.937 91.857) (end 177 92.92) (width 0.2) (layer "F.Cu") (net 17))
 (segment (start 148 100.54) (end 161.76 100.54) (width 0.2) (layer "F.Cu") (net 18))
 (segment (start 142.46 95) (end 148 100.54) (width 0.2) (layer "F.Cu") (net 18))
 (segment (start 184.13 90.38) (end 177 90.38) (width 0.2) (layer "B.Cu") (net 16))
 (segment (start 175.557 88.937) (end 177 90.38) (width 0.2) (layer "B.Cu") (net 16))
 (segment (start 137.38 95) (end 143.443 88.937) (width 0.2) (layer "B.Cu") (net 16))
 (segment (start 143.443 88.937) (end 175.557 88.937) (width 0.2) (layer "B.Cu") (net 16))
 (segment (start 188.75 95) (end 184.13 90.38) (width 0.2) (layer "B.Cu") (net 16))
 (segment (start 136.214 93.684) (end 142.058 87.84) (width 0.2) (layer "B.Cu") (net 2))
 (segment (start 153.358 113.46) (end 136.214 96.316) (width 0.2) (layer "B.Cu") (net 2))
 (segment (start 136.214 96.316) (end 136.214 93.684) (width 0.2) (layer "B.Cu") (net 2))
 (segment (start 138.19 132.46) (end 138.19 113.46) (width 0.2) (layer "B.Cu") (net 2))
 (segment (start 157.19 113.46) (end 153.358 113.46) (width 0.2) (layer "B.Cu") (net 2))
 (segment (start 142.058 87.84) (end 161.76 87.84) (width 0.2) (layer "B.Cu") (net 2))
 (segment (start 157.19 113.46) (end 138.19 113.46) (width 0.2) (layer "B.Cu") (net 2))
 (segment (start 176.11 108.11) (end 175 107) (width 0.2) (layer "B.Cu") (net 7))
 (segment (start 160.38 90.38) (end 161.76 90.38) (width 0.2) (layer "B.Cu") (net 7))
 (segment (start 160 90) (end 160.38 90.38) (width 0.2) (layer "B.Cu") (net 7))
 (segment (start 175 107) (end 159 107) (width 0.2) (layer "B.Cu") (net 7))
 (segment (start 159 90) (end 160 90) (width 0.2) (layer "B.Cu") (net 7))
 (segment (start 159 107) (end 159 90) (width 0.2) (layer "B.Cu") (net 7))
 (segment (start 176.11 113.46) (end 176.11 108.11) (width 0.2) (layer "B.Cu") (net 7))
 (segment (start 176.11 113.46) (end 176.11 132.46) (width 0.2) (layer "B.Cu") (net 7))
 (segment (start 157.19 132.46) (end 176.11 132.46) (width 0.2) (layer "B.Cu") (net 7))
 (segment (start 195.19 113.46) (end 190.73 109) (width 0.2) (layer "B.Cu") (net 5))
 (segment (start 177.84 109) (end 161.76 92.92) (width 0.2) (layer "B.Cu") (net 5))
 (segment (start 195.19 132.46) (end 195.19 113.46) (width 0.2) (layer "B.Cu") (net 5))
 (segment (start 190.73 109) (end 177.84 109) (width 0.2) (layer "B.Cu") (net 5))
 (segment (start 188.75 97.5) (end 183.17 103.08) (width 0.2) (layer "B.Cu") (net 21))
 (segment (start 183.17 103.08) (end 177 103.08) (width 0.2) (layer "B.Cu") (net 21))
 (segment (start 190.051 98.038892) (end 190.051 93.801) (width 0.2) (layer "B.Cu") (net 20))
 (segment (start 161.76 103.08) (end 160.697 102.017) (width 0.2) (layer "B.Cu") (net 20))
 (segment (start 161.31969 91.857) (end 164.27369 91.857) (width 0.2) (layer "B.Cu") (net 20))
 (segment (start 160.697 102.017) (end 160.697 92.47969) (width 0.2) (layer "B.Cu") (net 20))
 (segment (start 164.27369 91.857) (end 176.55969 104.143) (width 0.2) (layer "B.Cu") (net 20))
 (segment (start 176.55969 104.143) (end 183.946892 104.143) (width 0.2) (layer "B.Cu") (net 20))
 (segment (start 160.697 92.47969) (end 161.31969 91.857) (width 0.2) (layer "B.Cu") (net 20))
 (segment (start 190.051 93.801) (end 188.75 92.5) (width 0.2) (layer "B.Cu") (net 20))
 (segment (start 183.946892 104.143) (end 190.051 98.038892) (width 0.2) (layer "B.Cu") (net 20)))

